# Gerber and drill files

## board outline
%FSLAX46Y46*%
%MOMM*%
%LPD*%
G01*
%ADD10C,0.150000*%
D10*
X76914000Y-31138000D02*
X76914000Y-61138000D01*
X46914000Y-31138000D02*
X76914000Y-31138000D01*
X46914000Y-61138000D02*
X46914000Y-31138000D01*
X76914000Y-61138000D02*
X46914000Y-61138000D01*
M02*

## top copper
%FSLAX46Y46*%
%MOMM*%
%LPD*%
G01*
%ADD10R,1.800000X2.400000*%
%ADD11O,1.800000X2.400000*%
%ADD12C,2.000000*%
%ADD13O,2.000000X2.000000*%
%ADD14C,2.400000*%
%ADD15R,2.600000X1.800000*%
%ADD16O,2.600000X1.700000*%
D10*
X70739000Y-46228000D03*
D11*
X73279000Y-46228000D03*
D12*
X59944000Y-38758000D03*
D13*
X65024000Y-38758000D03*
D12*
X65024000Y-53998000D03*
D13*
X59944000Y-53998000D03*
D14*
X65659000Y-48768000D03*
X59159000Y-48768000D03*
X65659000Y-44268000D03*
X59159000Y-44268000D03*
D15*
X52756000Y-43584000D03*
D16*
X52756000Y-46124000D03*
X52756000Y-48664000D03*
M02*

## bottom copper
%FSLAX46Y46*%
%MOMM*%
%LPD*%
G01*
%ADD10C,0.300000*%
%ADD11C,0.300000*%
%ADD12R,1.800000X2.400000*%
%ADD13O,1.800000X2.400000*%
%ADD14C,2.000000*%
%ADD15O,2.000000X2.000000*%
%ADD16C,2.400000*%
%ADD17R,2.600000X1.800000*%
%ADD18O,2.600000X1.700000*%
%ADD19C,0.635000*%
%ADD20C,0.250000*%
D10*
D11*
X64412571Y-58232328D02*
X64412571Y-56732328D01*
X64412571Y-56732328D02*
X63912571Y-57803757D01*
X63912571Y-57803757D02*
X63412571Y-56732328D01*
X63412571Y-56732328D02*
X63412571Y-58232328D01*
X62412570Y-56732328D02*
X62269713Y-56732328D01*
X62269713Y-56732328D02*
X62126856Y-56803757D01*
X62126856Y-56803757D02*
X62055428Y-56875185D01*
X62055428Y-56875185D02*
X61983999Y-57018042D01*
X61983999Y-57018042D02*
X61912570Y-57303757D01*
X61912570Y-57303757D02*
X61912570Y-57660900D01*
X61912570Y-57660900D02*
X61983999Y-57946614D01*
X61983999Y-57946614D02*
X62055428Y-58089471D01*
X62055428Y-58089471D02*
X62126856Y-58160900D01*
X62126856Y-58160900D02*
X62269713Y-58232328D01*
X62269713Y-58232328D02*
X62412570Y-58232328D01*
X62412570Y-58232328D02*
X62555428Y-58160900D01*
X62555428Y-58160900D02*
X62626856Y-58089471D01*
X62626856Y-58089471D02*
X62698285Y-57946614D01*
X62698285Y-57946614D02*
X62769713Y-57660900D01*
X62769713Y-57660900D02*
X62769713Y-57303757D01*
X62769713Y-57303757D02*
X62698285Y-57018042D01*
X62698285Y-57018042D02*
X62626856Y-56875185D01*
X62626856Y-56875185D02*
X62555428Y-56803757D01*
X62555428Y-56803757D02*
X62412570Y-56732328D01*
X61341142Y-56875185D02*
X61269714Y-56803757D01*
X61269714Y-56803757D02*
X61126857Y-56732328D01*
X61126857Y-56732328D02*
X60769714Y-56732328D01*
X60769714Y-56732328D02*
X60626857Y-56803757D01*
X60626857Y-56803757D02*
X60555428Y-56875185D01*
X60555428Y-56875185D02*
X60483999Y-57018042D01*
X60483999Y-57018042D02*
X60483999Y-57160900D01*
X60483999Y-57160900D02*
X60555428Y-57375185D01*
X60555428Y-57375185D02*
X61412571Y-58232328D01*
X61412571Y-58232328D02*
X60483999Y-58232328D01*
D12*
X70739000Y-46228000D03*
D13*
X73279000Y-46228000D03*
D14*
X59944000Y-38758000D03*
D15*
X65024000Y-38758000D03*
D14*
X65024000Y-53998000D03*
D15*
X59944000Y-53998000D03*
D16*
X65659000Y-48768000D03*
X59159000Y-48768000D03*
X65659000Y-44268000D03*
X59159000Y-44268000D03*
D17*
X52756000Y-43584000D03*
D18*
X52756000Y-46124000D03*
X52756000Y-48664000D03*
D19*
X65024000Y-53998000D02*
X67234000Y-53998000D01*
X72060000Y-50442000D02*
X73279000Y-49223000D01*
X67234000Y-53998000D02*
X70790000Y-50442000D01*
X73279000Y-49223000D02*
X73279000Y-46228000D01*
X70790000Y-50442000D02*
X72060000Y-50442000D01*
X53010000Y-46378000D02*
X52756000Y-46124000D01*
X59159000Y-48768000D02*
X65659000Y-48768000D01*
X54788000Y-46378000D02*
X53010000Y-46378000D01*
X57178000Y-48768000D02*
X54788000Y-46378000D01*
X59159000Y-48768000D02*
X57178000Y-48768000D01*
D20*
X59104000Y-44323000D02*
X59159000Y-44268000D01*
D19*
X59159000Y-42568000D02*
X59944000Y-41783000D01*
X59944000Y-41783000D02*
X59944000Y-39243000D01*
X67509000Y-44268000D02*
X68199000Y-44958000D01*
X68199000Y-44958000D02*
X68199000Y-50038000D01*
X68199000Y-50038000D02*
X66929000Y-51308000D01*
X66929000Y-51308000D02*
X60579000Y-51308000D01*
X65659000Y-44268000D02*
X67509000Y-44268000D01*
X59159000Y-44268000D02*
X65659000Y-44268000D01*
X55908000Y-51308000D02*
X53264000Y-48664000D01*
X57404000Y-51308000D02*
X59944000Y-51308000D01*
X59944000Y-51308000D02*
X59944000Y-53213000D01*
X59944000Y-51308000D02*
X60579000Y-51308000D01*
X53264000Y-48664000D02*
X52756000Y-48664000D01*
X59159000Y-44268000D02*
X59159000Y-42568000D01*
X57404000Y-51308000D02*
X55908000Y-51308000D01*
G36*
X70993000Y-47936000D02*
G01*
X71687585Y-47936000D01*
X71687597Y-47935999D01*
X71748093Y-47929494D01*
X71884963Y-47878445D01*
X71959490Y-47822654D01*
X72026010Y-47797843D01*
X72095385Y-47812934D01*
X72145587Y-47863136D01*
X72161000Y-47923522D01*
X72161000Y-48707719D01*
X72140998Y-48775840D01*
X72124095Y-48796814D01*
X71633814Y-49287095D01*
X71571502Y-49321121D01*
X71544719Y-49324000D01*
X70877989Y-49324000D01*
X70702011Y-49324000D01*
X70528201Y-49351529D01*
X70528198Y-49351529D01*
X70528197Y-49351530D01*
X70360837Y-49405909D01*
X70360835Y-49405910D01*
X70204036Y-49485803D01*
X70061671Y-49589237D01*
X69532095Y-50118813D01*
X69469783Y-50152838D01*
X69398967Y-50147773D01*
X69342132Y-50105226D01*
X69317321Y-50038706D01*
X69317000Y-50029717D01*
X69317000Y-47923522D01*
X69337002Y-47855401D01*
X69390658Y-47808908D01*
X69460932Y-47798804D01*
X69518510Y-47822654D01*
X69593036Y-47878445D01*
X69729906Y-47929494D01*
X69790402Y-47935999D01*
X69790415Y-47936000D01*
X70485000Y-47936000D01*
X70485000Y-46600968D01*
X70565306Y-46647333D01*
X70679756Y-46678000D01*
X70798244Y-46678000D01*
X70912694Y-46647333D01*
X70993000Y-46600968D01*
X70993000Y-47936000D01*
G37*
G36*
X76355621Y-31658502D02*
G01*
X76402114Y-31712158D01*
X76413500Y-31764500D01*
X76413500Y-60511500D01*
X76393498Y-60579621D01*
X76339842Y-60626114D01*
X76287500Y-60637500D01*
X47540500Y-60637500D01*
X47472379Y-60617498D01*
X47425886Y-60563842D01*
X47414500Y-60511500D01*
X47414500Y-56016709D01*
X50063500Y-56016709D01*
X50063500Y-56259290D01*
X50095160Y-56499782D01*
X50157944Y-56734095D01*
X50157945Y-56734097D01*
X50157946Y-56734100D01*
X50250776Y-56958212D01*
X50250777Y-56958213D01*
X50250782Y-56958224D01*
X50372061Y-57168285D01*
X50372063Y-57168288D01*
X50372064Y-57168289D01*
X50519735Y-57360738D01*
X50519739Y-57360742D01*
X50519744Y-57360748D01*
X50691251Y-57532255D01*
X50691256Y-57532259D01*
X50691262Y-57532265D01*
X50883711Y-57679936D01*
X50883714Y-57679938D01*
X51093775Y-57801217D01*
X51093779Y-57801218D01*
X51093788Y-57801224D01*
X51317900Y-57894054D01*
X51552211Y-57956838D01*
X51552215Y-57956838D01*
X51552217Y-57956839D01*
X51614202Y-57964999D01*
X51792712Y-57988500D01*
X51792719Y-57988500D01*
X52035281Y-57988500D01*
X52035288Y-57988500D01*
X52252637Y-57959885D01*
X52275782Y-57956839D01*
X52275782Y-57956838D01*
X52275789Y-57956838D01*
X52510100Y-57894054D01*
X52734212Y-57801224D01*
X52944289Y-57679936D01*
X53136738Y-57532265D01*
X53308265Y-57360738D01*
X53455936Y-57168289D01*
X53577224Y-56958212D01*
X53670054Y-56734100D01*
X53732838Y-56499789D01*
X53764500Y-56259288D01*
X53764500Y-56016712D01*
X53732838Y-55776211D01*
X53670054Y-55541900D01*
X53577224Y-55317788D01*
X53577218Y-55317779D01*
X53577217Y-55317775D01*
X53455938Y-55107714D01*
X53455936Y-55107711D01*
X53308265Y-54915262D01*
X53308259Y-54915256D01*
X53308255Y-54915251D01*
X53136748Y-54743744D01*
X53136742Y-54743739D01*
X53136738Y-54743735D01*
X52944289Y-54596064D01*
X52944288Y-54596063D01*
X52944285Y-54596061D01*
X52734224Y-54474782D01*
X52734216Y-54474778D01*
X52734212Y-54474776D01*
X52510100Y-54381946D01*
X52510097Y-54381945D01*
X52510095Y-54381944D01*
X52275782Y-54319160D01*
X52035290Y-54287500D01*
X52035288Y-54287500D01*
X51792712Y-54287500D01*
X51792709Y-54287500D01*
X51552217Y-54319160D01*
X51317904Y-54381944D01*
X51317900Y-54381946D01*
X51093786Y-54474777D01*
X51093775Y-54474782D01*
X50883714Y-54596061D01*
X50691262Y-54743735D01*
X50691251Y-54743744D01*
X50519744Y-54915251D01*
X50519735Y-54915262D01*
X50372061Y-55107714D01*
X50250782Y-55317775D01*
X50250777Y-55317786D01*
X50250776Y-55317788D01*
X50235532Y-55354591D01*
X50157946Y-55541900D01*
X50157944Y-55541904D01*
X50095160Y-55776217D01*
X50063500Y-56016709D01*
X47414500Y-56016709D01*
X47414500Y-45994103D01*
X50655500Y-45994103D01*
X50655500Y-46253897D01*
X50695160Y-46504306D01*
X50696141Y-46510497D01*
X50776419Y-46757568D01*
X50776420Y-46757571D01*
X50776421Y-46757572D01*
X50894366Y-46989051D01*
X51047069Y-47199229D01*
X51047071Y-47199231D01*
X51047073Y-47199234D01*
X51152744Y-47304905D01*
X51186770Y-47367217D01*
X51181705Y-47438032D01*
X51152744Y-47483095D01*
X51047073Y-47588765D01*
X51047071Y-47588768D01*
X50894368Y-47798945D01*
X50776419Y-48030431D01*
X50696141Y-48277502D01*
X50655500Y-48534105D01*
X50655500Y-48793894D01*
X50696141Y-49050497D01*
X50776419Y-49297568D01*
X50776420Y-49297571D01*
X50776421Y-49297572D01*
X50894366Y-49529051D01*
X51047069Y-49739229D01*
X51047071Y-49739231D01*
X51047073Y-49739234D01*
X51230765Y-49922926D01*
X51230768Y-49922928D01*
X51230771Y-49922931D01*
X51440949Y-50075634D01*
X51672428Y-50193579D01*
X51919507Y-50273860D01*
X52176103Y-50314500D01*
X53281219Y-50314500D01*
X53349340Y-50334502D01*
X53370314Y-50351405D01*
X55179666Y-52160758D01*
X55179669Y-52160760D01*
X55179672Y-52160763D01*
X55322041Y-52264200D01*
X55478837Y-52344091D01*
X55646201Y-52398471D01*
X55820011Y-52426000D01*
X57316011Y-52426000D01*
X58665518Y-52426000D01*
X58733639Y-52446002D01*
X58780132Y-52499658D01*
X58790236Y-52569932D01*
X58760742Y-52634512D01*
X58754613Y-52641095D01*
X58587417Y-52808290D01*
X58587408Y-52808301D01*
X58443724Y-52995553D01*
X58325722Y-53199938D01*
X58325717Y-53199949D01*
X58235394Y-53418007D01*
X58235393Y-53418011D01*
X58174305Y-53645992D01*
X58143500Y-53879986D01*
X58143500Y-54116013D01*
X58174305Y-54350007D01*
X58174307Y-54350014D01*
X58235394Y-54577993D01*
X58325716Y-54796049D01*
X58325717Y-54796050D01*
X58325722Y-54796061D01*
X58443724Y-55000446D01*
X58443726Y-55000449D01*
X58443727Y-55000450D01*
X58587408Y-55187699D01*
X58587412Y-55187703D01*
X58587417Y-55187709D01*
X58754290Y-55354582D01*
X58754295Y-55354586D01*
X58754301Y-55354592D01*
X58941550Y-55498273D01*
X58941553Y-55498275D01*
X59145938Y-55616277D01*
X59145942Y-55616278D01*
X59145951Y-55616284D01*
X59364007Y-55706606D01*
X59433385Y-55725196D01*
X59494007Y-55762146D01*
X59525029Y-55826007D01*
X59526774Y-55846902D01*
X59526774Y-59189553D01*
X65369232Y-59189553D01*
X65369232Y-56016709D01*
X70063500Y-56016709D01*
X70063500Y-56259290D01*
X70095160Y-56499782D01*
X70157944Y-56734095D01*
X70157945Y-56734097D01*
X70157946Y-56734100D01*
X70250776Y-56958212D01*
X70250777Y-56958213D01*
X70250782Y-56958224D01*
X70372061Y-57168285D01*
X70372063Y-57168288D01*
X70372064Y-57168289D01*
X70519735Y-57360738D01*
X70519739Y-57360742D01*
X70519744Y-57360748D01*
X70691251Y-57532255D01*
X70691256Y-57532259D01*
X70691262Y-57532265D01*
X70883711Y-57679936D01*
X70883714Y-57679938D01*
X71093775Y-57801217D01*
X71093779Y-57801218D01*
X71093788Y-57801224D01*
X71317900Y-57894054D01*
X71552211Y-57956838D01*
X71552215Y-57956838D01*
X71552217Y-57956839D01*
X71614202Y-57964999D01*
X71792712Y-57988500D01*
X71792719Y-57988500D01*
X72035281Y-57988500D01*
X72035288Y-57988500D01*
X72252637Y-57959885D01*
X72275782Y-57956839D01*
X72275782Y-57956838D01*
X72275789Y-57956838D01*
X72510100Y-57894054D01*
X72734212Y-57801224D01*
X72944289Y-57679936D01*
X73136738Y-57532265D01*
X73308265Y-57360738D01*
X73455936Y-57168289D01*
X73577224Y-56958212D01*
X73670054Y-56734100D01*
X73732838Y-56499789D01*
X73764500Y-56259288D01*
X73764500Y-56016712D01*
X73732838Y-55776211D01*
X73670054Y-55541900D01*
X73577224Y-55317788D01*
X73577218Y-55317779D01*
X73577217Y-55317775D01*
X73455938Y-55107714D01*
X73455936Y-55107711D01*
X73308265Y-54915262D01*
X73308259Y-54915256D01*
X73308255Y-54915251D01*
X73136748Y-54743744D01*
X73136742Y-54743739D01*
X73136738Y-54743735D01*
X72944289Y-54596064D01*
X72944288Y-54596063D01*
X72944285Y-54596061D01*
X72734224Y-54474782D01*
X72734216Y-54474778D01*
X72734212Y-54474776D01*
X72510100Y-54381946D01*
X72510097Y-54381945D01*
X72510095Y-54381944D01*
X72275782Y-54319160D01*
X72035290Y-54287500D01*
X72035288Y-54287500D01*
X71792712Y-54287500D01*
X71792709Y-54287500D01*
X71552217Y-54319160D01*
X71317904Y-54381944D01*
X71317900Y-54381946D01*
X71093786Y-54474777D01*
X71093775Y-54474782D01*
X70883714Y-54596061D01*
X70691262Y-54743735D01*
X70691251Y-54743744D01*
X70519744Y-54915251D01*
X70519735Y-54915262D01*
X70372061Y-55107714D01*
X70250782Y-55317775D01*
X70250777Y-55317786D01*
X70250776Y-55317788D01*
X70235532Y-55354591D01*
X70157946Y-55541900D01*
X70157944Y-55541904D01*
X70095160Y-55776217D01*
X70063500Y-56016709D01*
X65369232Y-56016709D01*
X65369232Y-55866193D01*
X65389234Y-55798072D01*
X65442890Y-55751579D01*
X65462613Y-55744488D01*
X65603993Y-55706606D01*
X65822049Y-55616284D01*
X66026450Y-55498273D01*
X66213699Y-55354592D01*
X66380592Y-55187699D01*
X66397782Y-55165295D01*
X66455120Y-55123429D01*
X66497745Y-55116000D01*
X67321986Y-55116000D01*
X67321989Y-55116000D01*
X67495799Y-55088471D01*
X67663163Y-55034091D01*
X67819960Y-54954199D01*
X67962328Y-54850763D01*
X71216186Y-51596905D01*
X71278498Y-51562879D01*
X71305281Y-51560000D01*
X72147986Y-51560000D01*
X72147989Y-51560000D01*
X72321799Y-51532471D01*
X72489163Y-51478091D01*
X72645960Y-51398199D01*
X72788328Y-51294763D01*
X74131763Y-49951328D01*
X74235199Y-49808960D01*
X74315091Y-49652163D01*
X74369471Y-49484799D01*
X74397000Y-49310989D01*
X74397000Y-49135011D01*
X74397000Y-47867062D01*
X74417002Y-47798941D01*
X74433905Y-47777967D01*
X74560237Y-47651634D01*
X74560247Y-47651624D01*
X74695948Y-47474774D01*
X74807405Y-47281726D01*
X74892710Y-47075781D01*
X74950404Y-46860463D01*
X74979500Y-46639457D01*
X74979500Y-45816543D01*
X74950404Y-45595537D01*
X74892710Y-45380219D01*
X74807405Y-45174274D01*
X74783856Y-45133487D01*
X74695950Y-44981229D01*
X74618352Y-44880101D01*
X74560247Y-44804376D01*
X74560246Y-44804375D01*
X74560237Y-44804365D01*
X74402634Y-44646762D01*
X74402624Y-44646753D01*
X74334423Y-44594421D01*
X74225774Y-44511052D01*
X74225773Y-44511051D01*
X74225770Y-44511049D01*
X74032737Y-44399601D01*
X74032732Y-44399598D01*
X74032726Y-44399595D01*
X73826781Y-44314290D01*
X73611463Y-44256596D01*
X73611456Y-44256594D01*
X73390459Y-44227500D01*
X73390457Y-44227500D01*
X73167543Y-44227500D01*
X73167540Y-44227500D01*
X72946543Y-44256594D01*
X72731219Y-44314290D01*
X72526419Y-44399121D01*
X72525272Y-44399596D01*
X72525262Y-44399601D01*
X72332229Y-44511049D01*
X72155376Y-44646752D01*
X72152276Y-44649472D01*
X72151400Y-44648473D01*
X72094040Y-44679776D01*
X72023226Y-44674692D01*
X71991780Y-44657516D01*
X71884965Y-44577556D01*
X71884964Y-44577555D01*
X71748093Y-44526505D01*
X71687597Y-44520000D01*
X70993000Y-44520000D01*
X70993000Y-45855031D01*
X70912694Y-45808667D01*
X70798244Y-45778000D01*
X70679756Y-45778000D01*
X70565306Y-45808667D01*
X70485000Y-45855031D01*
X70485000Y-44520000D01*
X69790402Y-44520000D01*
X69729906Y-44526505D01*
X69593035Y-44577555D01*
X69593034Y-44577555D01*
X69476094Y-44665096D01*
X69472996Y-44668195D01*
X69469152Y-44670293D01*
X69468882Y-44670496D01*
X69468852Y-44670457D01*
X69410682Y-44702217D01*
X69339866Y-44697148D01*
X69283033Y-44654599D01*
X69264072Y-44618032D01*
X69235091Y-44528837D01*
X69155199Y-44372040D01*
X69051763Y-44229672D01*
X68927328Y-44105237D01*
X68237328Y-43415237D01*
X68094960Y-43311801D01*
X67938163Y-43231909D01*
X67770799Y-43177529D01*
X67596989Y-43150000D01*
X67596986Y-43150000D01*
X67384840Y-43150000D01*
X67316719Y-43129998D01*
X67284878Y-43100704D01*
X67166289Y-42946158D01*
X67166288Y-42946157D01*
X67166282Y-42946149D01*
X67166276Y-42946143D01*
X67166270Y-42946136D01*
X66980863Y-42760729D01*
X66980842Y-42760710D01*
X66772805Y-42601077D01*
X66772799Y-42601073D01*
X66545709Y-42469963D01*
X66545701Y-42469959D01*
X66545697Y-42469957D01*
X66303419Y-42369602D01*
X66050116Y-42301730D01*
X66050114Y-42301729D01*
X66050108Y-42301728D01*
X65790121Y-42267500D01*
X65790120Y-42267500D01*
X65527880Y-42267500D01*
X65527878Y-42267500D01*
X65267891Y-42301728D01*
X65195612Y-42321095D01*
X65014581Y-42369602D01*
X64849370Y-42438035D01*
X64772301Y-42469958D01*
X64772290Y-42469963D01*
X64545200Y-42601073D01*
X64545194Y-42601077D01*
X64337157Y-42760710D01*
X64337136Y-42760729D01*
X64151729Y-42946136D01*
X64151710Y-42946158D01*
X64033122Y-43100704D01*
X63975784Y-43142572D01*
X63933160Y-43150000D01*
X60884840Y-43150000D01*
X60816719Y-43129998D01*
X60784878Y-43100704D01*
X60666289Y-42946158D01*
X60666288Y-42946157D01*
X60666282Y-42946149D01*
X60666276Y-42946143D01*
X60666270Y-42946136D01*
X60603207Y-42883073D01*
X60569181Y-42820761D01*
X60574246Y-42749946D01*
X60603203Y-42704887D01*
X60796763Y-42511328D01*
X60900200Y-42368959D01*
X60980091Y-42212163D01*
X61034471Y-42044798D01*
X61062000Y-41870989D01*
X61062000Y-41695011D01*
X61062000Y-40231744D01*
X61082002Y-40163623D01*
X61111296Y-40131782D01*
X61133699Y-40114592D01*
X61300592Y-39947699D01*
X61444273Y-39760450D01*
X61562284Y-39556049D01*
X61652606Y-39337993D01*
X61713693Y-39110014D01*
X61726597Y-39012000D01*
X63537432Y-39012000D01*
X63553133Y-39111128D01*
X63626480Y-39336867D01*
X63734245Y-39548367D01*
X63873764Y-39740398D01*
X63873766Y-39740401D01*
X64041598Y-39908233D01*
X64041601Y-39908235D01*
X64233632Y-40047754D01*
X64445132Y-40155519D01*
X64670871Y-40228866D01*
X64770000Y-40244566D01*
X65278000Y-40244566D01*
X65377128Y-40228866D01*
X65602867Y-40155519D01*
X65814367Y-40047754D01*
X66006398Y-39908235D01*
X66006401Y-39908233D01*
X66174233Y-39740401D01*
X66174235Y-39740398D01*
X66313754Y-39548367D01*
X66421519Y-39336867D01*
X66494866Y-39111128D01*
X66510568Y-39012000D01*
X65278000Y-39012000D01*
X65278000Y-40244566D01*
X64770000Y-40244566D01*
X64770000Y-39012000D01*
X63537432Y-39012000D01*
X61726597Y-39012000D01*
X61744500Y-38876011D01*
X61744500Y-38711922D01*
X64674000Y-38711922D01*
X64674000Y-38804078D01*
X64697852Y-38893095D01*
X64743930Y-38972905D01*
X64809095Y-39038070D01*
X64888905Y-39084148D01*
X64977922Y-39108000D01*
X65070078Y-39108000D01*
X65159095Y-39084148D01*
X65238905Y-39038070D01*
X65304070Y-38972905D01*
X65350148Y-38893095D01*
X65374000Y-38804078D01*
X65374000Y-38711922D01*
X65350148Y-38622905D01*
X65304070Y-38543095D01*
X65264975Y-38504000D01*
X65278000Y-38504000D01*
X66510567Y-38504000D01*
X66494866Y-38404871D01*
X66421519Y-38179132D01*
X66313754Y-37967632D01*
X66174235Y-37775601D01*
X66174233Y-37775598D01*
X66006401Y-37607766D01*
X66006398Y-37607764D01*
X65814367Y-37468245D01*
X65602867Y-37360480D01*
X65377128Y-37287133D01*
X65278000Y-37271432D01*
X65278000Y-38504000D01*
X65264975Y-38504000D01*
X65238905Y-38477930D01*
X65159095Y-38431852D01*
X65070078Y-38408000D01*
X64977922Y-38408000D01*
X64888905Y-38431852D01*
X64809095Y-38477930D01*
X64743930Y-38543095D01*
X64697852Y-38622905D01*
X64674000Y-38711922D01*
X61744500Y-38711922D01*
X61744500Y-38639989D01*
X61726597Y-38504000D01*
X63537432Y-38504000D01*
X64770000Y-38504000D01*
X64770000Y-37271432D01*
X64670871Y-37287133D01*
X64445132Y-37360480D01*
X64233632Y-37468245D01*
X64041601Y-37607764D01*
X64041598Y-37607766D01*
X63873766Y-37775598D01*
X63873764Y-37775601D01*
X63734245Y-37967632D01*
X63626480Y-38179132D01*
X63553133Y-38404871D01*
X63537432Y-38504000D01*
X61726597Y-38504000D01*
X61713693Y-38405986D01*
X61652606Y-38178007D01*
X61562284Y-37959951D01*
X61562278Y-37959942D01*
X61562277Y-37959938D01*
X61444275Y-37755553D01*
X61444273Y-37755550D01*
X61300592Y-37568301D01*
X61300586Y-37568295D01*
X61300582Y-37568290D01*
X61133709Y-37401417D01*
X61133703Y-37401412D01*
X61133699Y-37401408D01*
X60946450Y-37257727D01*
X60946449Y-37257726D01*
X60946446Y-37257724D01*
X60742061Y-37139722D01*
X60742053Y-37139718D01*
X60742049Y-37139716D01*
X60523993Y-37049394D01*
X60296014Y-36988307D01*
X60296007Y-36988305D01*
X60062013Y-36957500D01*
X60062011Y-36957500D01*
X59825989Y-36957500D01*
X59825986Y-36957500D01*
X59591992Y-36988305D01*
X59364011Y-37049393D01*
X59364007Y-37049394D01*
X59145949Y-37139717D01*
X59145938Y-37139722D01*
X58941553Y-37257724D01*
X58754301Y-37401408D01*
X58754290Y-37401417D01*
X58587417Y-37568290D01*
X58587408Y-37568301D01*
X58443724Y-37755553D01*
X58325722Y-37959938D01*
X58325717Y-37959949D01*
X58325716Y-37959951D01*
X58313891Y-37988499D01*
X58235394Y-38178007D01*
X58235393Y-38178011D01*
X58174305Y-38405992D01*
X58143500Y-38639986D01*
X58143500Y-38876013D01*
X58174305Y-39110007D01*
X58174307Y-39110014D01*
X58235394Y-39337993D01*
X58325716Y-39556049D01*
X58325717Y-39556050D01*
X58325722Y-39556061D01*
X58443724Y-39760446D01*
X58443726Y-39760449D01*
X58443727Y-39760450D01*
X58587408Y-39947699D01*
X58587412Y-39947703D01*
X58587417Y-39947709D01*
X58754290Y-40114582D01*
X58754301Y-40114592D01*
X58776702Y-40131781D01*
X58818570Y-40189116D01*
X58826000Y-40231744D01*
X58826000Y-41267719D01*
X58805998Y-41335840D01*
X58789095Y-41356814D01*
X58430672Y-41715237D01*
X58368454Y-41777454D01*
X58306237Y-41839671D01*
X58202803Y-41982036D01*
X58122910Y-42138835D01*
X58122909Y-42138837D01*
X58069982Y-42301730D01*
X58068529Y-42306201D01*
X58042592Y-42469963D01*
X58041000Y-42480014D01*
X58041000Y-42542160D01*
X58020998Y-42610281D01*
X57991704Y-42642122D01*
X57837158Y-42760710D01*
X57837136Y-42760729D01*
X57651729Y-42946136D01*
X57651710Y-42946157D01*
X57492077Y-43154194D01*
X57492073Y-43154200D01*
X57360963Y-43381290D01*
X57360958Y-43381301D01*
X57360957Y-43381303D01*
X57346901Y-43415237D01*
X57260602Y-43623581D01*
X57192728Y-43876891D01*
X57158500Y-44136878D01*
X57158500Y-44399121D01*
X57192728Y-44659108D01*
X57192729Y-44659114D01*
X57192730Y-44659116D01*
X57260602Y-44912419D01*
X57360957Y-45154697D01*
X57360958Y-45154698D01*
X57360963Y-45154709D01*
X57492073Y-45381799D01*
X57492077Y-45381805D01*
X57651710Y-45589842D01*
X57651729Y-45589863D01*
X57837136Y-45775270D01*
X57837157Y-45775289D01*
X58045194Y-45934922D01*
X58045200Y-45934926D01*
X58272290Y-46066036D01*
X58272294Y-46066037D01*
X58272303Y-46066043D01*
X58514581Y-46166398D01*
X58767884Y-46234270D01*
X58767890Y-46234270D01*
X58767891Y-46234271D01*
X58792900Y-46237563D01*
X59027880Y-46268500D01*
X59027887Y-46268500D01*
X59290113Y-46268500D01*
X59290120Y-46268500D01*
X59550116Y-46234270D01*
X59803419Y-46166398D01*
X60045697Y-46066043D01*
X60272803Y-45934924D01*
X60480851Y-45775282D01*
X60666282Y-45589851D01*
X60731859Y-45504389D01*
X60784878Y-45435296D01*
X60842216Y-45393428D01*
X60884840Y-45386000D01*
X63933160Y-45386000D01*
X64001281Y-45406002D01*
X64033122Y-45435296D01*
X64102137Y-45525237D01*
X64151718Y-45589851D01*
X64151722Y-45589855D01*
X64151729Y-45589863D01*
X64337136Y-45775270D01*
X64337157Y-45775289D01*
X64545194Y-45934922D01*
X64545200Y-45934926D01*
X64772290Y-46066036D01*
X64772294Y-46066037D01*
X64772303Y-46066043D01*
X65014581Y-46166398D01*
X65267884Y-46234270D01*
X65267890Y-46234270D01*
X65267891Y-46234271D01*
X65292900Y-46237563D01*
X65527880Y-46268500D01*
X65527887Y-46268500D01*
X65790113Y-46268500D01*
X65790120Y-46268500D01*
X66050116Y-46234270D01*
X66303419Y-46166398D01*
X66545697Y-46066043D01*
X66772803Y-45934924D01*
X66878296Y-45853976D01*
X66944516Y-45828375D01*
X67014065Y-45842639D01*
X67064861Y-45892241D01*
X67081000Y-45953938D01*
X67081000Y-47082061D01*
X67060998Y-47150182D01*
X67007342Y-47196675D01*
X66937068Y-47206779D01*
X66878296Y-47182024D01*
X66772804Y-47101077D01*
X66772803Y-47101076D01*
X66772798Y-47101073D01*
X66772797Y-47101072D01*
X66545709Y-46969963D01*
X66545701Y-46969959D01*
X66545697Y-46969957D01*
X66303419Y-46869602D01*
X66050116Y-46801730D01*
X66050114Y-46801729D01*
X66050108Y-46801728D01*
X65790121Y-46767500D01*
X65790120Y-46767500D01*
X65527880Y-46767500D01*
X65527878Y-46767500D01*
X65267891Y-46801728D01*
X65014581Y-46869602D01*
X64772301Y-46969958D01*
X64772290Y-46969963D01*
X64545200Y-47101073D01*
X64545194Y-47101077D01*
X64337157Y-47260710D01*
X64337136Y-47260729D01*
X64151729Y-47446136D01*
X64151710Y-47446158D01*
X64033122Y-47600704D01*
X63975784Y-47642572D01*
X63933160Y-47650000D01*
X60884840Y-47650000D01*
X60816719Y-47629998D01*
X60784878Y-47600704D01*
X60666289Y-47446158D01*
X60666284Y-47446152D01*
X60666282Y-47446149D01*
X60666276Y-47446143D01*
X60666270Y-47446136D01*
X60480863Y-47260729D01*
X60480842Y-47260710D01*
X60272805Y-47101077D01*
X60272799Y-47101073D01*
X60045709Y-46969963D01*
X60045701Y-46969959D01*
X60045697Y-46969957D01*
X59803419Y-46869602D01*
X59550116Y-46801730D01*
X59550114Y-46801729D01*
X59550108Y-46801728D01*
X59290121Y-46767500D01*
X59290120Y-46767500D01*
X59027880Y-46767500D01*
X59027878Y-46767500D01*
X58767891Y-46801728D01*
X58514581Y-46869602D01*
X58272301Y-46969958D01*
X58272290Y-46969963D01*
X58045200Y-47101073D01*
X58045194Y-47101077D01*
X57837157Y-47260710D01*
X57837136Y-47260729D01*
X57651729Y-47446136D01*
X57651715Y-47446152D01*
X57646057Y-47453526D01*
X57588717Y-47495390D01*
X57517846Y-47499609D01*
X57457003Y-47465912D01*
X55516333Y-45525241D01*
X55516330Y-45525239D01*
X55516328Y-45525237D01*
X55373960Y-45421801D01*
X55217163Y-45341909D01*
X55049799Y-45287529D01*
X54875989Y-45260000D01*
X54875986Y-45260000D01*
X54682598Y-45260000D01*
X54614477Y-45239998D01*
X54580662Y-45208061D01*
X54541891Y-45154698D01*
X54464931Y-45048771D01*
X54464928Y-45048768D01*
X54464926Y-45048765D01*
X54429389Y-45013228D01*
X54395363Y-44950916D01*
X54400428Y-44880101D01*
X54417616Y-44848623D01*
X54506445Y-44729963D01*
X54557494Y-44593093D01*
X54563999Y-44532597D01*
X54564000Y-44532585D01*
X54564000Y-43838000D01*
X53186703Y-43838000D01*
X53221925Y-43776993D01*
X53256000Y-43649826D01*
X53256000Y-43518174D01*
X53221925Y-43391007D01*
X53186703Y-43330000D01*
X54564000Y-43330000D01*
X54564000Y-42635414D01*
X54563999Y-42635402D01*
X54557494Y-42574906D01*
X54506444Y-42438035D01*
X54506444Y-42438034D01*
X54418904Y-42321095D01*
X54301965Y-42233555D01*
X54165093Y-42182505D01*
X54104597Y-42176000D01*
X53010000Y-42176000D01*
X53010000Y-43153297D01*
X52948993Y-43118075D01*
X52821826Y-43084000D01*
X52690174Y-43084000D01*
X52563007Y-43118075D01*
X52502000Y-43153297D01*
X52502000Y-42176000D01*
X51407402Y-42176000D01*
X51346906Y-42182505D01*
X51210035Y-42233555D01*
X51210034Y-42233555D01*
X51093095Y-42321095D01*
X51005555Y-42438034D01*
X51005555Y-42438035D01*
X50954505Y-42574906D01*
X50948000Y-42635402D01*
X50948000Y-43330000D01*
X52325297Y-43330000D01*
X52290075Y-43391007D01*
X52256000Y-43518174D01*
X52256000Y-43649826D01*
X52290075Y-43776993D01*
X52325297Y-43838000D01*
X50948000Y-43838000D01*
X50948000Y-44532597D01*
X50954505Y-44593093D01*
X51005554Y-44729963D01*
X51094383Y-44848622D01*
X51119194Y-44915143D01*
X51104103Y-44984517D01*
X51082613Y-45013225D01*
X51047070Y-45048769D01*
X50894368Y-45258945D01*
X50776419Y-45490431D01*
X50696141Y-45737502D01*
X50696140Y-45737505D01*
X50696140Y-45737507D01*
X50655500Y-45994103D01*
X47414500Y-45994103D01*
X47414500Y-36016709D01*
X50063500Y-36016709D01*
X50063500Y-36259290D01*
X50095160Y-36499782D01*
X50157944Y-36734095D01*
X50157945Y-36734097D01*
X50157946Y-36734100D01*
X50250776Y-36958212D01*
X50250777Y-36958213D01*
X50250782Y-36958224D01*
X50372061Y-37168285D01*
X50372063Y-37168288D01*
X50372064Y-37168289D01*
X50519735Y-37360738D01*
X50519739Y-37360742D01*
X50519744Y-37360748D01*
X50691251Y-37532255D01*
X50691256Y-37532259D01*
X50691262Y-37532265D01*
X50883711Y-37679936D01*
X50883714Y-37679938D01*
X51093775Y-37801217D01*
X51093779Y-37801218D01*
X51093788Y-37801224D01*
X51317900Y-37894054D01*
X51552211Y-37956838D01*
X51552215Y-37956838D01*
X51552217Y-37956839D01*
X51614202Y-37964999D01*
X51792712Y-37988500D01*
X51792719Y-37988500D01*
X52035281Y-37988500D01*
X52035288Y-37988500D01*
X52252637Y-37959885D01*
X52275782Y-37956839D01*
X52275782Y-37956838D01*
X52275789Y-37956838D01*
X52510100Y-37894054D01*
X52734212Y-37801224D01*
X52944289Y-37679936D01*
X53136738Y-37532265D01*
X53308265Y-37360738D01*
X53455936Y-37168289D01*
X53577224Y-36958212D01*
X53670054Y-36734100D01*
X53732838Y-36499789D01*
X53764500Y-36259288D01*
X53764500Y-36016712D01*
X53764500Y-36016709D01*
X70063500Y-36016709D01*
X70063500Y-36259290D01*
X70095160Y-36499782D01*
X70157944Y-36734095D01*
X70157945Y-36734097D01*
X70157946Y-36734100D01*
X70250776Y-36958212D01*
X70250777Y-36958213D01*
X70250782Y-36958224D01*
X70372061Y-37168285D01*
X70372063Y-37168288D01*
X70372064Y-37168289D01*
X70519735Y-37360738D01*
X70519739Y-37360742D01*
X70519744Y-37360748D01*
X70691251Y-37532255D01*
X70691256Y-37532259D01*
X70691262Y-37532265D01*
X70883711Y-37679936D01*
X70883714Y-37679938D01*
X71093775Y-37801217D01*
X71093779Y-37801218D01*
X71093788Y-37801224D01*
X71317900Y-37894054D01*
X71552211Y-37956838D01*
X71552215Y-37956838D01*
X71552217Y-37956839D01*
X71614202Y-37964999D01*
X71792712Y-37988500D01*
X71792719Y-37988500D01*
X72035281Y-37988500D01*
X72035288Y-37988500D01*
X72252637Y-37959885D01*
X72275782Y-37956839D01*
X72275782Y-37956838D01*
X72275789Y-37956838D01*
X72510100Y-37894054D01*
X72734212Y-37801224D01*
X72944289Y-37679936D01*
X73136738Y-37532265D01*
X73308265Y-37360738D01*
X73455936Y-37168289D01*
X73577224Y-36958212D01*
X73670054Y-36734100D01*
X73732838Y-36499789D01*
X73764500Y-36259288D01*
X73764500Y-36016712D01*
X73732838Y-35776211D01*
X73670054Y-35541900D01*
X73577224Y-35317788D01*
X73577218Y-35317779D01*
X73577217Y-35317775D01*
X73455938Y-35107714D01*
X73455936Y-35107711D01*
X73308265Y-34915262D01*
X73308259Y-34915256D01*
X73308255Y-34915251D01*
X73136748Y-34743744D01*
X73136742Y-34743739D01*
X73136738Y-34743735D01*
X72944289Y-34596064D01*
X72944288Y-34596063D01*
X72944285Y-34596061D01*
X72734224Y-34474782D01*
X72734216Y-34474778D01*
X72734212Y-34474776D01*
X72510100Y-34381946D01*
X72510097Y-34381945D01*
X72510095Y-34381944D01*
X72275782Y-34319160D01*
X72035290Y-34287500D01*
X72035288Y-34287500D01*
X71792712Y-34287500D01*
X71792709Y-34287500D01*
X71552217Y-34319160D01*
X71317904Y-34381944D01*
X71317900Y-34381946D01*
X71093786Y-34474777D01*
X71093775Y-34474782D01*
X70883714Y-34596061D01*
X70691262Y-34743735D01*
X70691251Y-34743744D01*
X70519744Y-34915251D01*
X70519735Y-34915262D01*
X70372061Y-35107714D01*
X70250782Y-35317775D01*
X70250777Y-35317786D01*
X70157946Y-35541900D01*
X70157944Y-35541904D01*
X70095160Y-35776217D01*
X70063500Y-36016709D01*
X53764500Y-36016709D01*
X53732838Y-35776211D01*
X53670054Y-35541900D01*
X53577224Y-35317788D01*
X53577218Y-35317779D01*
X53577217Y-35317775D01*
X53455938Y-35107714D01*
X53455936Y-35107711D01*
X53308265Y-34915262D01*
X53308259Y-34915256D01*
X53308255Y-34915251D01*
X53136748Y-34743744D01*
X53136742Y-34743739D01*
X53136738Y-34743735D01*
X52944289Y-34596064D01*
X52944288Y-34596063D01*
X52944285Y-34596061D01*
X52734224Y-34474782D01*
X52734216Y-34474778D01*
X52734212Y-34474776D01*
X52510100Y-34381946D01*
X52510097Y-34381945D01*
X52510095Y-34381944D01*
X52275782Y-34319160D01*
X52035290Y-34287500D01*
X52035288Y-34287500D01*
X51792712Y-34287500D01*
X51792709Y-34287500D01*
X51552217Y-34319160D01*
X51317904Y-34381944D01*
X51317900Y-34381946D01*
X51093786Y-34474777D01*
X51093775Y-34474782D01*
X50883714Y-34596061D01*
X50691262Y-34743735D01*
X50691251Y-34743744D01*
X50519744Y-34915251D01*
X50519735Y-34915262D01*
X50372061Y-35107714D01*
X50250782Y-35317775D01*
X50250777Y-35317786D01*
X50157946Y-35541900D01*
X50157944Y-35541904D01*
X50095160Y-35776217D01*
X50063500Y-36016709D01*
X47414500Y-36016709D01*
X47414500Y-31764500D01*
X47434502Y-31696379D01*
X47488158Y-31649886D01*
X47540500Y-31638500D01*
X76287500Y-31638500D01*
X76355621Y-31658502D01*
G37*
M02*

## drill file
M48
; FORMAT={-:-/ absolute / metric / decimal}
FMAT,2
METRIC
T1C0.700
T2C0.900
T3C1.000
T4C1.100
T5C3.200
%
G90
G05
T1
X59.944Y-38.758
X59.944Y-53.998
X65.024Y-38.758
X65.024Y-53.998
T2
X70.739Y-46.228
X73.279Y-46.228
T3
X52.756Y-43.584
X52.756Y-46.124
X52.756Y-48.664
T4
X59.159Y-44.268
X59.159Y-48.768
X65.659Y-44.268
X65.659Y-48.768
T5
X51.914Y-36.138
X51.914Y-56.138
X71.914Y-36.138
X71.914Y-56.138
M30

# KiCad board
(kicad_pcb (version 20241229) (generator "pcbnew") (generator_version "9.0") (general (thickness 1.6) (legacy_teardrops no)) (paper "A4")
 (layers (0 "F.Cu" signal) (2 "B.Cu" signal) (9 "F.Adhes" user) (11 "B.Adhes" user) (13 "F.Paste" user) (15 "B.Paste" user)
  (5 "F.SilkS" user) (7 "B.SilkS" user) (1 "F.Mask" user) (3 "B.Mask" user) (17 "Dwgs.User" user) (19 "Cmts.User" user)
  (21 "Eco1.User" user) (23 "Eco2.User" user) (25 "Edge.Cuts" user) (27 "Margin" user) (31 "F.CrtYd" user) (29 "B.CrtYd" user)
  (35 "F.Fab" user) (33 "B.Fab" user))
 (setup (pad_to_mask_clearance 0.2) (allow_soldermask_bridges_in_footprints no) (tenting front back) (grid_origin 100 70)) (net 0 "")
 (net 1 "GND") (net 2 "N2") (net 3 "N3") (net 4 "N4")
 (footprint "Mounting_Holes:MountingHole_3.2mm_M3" (layer "F.Cu") (at 51.914 36.138)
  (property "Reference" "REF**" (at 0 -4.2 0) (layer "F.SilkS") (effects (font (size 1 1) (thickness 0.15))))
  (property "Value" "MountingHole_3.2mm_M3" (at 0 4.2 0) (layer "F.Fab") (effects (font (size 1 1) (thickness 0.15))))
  (pad "" np_thru_hole circle (at 0 0) (size 3.2 3.2) (drill 3.2) (layers "*.Cu" "*.Mask")))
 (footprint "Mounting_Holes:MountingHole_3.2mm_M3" (layer "F.Cu") (at 71.914 36.138)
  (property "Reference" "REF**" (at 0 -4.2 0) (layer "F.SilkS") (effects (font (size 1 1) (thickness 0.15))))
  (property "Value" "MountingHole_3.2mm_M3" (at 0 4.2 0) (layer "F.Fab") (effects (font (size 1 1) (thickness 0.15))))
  (pad "" np_thru_hole circle (at 0 0) (size 3.2 3.2) (drill 3.2) (layers "*.Cu" "*.Mask")))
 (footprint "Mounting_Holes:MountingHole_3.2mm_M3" (layer "F.Cu") (at 71.914 56.138)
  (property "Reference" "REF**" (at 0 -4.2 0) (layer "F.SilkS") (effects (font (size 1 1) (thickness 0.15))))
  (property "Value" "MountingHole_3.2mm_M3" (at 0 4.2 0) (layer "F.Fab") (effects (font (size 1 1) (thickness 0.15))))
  (pad "" np_thru_hole circle (at 0 0) (size 3.2 3.2) (drill 3.2) (layers "*.Cu" "*.Mask")))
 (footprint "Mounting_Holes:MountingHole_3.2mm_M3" (layer "F.Cu") (at 51.914 56.138)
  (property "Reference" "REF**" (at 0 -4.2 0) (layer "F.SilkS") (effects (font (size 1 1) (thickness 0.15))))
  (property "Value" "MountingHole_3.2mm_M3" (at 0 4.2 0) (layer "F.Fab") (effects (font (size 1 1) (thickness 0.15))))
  (pad "" np_thru_hole circle (at 0 0) (size 3.2 3.2) (drill 3.2) (layers "*.Cu" "*.Mask")))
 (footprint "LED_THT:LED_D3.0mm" (layer "F.Cu") (at 70.739 46.228)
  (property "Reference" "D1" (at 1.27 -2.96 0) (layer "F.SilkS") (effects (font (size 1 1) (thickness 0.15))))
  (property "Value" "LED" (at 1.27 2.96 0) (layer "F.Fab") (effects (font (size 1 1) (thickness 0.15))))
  (pad "1" thru_hole rect (at 0 0) (size 1.8 2.4) (drill 0.9) (layers "*.Cu" "*.Mask") (remove_unused_layers no) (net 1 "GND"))
  (pad "2" thru_hole oval (at 2.54 0) (size 1.8 2.4) (drill 0.9) (layers "*.Cu" "*.Mask") (remove_unused_layers no) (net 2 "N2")))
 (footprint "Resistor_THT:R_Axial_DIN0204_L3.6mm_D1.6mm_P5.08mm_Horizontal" (layer "F.Cu") (at 59.944 38.758)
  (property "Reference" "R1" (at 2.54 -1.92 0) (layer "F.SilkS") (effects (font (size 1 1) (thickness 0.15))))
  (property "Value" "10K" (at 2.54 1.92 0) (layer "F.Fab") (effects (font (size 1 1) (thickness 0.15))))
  (pad "1" thru_hole circle (at 0 0) (size 2 2) (drill 0.7) (layers "*.Cu" "*.Mask") (remove_unused_layers no) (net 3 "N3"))
  (pad "2" thru_hole oval (at 5.08 0) (size 2 2) (drill 0.7) (layers "*.Cu" "*.Mask") (remove_unused_layers no) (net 1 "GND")))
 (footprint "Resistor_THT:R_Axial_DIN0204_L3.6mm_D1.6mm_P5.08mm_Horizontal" (layer "F.Cu") (at 65.024 53.998 180)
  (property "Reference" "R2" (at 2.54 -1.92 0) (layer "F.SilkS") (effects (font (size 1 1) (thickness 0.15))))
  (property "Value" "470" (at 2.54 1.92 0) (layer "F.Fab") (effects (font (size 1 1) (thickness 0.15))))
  (pad "1" thru_hole circle (at 0 0 180) (size 2 2) (drill 0.7) (layers "*.Cu" "*.Mask") (remove_unused_layers no) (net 2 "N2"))
  (pad "2" thru_hole oval (at 5.08 0 180) (size 2 2) (drill 0.7) (layers "*.Cu" "*.Mask") (remove_unused_layers no) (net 3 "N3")))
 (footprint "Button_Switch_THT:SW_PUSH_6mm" (layer "F.Cu") (at 65.659 48.768 180)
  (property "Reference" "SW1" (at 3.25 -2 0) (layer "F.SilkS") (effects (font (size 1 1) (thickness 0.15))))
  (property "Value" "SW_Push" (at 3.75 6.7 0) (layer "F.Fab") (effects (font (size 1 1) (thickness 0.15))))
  (pad "1" thru_hole circle (at 0 0 270) (size 2.4 2.4) (drill 1.1) (layers "*.Cu" "*.Mask") (remove_unused_layers no) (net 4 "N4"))
  (pad "1" thru_hole circle (at 6.5 0 270) (size 2.4 2.4) (drill 1.1) (layers "*.Cu" "*.Mask") (remove_unused_layers no) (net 4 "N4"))
  (pad "2" thru_hole circle (at 0 4.5 270) (size 2.4 2.4) (drill 1.1) (layers "*.Cu" "*.Mask") (remove_unused_layers no) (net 3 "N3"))
  (pad "2" thru_hole circle (at 6.5 4.5 270) (size 2.4 2.4) (drill 1.1) (layers "*.Cu" "*.Mask") (remove_unused_layers no) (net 3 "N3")))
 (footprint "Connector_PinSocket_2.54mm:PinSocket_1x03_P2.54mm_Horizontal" (layer "F.Cu") (at 52.756 43.584)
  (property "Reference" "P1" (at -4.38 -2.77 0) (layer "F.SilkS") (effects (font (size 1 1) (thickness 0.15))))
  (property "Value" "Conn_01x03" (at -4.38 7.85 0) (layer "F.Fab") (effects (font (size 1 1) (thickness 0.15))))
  (pad "1" thru_hole rect (at 0 0) (size 2.6 1.8) (drill 1) (layers "*.Cu" "*.Mask") (remove_unused_layers no) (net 1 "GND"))
  (pad "2" thru_hole oval (at 0 2.54) (size 2.6 1.7) (drill 1) (layers "*.Cu" "*.Mask") (remove_unused_layers no) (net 4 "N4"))
  (pad "3" thru_hole oval (at 0 5.08) (size 2.6 1.7) (drill 1) (layers "*.Cu" "*.Mask") (remove_unused_layers no) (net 3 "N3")))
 (gr_line (start 76.914 31.138) (end 76.914 61.138) (stroke (width 0.15) (type solid)) (layer "Edge.Cuts"))
 (gr_line (start 46.914 31.138) (end 76.914 31.138) (stroke (width 0.15) (type solid)) (layer "Edge.Cuts"))
 (gr_line (start 46.914 61.138) (end 46.914 31.138) (stroke (width 0.15) (type solid)) (layer "Edge.Cuts"))
 (gr_line (start 76.914 61.138) (end 46.914 61.138) (stroke (width 0.15) (type solid)) (layer "Edge.Cuts"))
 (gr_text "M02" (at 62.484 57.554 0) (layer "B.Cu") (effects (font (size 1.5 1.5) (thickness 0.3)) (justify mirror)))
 (segment (start 65.024 53.998) (end 67.234 53.998) (width 0.635) (layer "B.Cu") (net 2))
 (segment (start 72.06 50.442) (end 73.279 49.223) (width 0.635) (layer "B.Cu") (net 2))
 (segment (start 67.234 53.998) (end 70.79 50.442) (width 0.635) (layer "B.Cu") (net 2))
 (segment (start 73.279 49.223) (end 73.279 46.228) (width 0.635) (layer "B.Cu") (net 2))
 (segment (start 70.79 50.442) (end 72.06 50.442) (width 0.635) (layer "B.Cu") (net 2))
 (segment (start 53.01 46.378) (end 52.756 46.124) (width 0.635) (layer "B.Cu") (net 4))
 (segment (start 59.159 48.768) (end 65.659 48.768) (width 0.635) (layer "B.Cu") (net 4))
 (segment (start 54.788 46.378) (end 53.01 46.378) (width 0.635) (layer "B.Cu") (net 4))
 (segment (start 57.178 48.768) (end 54.788 46.378) (width 0.635) (layer "B.Cu") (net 4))
 (segment (start 59.159 48.768) (end 57.178 48.768) (width 0.635) (layer "B.Cu") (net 4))
 (segment (start 59.104 44.323) (end 59.159 44.268) (width 0.25) (layer "B.Cu") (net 3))
 (segment (start 59.159 42.568) (end 59.944 41.783) (width 0.635) (layer "B.Cu") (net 3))
 (segment (start 59.944 41.783) (end 59.944 39.243) (width 0.635) (layer "B.Cu") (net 3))
 (segment (start 67.509 44.268) (end 68.199 44.958) (width 0.635) (layer "B.Cu") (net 3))
 (segment (start 68.199 44.958) (end 68.199 50.038) (width 0.635) (layer "B.Cu") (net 3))
 (segment (start 68.199 50.038) (end 66.929 51.308) (width 0.635) (layer "B.Cu") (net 3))
 (segment (start 66.929 51.308) (end 60.579 51.308) (width 0.635) (layer "B.Cu") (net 3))
 (segment (start 65.659 44.268) (end 67.509 44.268) (width 0.635) (layer "B.Cu") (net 3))
 (segment (start 59.159 44.268) (end 65.659 44.268) (width 0.635) (layer "B.Cu") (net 3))
 (segment (start 55.908 51.308) (end 53.264 48.664) (width 0.635) (layer "B.Cu") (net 3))
 (segment (start 57.404 51.308) (end 59.944 51.308) (width 0.635) (layer "B.Cu") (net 3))
 (segment (start 59.944 51.308) (end 59.944 53.213) (width 0.635) (layer "B.Cu") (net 3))
 (segment (start 59.944 51.308) (end 60.579 51.308) (width 0.635) (layer "B.Cu") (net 3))
 (segment (start 53.264 48.664) (end 52.756 48.664) (width 0.635) (layer "B.Cu") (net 3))
 (segment (start 59.159 44.268) (end 59.159 42.568) (width 0.635) (layer "B.Cu") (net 3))
 (segment (start 57.404 51.308) (end 55.908 51.308) (width 0.635) (layer "B.Cu") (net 3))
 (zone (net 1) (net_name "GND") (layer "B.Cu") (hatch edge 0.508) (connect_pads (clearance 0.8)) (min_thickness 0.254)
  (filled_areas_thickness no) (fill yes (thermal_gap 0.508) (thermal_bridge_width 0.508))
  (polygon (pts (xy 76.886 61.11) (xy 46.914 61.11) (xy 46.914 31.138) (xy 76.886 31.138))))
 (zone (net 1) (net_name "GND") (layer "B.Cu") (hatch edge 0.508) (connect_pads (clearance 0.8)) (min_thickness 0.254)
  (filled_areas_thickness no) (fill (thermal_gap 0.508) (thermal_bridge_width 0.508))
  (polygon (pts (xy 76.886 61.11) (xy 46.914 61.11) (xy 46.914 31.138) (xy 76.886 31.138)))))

